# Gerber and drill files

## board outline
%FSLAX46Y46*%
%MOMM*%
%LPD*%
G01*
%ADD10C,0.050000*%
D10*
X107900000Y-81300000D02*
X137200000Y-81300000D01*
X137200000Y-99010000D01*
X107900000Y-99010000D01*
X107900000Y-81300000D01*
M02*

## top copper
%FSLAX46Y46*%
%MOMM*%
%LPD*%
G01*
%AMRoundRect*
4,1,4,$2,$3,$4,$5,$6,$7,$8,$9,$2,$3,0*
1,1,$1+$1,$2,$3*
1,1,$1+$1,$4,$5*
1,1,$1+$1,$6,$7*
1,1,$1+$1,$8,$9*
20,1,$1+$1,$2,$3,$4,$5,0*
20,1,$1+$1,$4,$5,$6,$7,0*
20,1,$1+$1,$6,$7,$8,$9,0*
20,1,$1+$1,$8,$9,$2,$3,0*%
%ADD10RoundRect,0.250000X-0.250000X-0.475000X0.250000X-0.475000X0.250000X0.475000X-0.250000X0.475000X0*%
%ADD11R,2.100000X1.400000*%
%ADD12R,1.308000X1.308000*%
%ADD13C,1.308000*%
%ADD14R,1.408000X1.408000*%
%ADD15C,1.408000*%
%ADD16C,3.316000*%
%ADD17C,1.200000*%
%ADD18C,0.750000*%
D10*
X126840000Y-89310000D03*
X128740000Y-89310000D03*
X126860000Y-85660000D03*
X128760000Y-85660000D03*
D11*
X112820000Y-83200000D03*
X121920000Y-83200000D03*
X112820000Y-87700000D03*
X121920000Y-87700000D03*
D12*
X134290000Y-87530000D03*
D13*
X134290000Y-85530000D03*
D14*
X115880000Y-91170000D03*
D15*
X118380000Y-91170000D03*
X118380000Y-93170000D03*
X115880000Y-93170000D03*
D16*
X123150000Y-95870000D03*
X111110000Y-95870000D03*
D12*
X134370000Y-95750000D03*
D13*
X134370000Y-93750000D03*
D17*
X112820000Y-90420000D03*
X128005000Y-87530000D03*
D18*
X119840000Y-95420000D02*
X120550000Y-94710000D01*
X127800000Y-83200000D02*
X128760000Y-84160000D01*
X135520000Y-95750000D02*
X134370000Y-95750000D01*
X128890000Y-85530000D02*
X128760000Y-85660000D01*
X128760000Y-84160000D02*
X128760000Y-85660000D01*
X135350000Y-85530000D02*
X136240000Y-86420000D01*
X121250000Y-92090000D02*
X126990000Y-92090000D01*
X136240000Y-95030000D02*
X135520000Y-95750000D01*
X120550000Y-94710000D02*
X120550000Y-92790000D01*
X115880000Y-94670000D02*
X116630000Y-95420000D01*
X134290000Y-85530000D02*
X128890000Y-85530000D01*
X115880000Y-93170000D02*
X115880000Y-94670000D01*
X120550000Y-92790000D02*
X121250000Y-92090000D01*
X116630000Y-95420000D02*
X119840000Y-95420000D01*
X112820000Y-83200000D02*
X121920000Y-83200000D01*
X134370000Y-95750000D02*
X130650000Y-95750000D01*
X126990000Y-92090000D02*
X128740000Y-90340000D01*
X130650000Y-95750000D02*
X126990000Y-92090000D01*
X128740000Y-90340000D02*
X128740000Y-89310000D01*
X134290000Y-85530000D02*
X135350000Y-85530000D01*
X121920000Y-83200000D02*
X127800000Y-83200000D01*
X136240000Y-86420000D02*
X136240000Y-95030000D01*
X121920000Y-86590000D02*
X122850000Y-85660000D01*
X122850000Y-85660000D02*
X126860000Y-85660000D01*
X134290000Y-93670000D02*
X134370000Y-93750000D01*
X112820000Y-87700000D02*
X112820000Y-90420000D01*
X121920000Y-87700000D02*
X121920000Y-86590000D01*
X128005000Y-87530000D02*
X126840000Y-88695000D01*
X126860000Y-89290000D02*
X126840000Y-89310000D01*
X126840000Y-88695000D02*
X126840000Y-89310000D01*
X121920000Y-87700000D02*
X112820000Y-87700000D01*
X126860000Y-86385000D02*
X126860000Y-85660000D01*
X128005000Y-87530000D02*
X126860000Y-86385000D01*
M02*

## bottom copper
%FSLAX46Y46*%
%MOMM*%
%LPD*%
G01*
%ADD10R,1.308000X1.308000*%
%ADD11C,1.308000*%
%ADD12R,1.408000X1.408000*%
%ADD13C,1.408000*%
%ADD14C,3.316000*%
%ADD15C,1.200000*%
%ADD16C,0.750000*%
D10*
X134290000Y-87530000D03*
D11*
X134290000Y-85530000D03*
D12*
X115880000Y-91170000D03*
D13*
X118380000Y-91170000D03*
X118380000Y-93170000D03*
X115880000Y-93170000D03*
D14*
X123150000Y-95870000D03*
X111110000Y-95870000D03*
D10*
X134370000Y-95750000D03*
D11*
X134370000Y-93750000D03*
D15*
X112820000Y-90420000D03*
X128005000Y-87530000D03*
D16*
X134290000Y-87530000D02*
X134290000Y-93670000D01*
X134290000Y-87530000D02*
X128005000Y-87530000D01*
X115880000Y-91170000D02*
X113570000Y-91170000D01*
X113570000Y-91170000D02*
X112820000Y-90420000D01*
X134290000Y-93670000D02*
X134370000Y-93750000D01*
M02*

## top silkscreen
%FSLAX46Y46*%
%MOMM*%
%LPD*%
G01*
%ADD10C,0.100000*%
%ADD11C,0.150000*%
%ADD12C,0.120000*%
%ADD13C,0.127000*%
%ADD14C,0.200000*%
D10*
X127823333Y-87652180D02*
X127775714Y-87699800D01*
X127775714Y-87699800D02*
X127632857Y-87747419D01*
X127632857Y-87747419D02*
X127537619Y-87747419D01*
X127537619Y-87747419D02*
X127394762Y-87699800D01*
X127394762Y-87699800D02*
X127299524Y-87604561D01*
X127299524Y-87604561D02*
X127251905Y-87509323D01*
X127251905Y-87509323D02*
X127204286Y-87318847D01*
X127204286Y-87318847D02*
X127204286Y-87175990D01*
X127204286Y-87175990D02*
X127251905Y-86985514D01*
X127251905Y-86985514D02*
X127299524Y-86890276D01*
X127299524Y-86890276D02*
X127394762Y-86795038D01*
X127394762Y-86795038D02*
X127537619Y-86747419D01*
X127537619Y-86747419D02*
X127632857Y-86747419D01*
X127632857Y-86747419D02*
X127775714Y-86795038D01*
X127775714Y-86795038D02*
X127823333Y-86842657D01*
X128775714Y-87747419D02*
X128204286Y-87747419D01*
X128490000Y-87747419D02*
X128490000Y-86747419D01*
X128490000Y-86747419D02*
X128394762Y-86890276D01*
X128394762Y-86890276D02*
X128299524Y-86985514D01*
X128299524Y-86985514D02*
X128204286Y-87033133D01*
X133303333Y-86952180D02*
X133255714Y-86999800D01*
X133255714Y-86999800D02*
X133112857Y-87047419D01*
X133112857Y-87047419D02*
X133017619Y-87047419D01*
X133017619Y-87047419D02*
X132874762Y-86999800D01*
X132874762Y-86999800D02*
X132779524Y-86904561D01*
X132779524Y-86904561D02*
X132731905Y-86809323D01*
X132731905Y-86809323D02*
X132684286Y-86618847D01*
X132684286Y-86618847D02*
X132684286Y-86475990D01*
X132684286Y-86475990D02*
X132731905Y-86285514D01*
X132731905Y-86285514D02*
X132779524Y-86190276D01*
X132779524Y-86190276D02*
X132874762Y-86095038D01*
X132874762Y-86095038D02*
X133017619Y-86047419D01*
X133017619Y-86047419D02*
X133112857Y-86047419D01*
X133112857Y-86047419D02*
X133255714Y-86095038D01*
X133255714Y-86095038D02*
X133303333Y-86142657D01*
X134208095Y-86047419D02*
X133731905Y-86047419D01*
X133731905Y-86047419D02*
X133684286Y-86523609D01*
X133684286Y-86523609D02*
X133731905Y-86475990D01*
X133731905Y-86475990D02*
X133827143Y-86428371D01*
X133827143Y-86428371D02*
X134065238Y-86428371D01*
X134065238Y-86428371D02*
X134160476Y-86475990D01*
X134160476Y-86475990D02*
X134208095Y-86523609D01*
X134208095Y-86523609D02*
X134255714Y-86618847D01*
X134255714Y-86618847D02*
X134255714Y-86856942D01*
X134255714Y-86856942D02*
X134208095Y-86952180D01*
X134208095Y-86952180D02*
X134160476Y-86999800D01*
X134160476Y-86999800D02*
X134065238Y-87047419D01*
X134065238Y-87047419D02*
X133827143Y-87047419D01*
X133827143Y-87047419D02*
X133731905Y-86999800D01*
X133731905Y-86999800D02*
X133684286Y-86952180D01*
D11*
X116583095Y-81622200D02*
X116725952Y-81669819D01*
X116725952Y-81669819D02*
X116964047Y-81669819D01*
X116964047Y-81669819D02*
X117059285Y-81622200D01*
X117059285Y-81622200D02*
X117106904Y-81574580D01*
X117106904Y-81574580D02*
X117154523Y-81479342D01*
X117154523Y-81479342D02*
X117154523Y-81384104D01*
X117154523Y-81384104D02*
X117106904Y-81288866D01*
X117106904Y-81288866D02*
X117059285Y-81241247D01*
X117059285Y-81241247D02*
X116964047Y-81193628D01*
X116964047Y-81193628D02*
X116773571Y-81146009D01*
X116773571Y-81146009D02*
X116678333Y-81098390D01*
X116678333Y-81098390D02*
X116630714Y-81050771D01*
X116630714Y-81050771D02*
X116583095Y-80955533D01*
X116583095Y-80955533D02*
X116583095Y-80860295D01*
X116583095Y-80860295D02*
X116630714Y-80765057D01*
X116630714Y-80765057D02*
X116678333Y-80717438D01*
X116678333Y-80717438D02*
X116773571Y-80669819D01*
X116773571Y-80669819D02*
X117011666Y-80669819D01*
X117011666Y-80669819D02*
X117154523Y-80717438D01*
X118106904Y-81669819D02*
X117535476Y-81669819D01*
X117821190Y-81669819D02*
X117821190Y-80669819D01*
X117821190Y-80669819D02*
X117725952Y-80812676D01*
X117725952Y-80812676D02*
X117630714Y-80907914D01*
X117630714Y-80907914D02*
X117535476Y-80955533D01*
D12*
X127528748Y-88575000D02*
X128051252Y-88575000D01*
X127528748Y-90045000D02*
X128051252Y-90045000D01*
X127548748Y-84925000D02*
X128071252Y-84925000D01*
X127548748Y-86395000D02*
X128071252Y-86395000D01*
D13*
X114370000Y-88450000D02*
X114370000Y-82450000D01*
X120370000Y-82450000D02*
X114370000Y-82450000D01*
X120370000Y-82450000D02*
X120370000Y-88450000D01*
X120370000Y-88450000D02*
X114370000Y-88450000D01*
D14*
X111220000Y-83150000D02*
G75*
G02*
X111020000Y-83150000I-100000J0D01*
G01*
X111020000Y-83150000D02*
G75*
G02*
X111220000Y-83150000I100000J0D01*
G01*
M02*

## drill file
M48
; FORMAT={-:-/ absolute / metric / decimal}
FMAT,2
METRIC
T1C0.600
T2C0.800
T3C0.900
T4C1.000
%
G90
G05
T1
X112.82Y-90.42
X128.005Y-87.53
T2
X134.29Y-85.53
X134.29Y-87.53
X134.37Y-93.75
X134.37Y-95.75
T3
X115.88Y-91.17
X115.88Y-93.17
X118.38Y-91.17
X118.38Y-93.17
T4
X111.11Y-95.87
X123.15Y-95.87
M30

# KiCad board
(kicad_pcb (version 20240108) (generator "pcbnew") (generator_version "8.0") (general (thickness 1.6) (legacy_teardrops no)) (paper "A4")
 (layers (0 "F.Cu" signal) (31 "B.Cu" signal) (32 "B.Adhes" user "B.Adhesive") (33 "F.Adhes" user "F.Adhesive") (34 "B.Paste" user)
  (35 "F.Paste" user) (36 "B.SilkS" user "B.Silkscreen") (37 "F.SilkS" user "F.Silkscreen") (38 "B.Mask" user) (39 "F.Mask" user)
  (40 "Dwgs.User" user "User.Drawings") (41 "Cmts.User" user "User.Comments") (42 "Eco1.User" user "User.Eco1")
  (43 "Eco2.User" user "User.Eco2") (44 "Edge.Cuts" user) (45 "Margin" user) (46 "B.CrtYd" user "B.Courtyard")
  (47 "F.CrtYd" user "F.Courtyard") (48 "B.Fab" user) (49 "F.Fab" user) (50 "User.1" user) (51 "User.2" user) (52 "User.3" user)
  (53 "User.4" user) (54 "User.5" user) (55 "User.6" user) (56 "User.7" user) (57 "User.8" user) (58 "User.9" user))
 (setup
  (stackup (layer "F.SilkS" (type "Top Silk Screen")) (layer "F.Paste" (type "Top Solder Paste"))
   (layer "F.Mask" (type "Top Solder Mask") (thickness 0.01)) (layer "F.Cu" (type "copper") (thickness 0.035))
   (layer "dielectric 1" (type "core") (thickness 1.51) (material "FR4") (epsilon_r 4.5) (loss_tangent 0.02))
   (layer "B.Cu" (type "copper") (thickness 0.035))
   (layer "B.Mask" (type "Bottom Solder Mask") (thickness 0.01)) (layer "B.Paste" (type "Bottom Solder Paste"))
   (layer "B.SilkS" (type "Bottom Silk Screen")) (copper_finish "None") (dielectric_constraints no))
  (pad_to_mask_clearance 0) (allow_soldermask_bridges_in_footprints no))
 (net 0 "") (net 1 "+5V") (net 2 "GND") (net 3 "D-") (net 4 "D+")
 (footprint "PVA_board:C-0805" (layer "F.Cu") (at 127.79 89.31)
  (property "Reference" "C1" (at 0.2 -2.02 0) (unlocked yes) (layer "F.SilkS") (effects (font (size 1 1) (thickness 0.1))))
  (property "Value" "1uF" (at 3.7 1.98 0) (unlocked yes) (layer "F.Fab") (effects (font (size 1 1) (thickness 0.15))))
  (fp_line (start -0.261252 -0.735) (end 0.261252 -0.735) (stroke (width 0.12) (type solid)) (layer "F.SilkS"))
  (fp_line (start -0.261252 0.735) (end 0.261252 0.735) (stroke (width 0.12) (type solid)) (layer "F.SilkS"))
  (pad "1" smd roundrect (at -0.95 0) (size 1 1.45) (layers "F.Cu" "F.Paste" "F.Mask") (roundrect_rratio 0.25) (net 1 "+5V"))
  (pad "2" smd roundrect (at 0.95 0) (size 1 1.45) (layers "F.Cu" "F.Paste" "F.Mask") (roundrect_rratio 0.25) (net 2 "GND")))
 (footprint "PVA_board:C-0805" (layer "F.Cu") (at 127.81 85.66)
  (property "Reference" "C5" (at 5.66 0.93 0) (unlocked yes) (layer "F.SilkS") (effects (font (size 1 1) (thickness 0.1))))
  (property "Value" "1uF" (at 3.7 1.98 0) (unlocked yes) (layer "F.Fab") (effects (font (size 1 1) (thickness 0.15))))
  (fp_line (start -0.261252 -0.735) (end 0.261252 -0.735) (stroke (width 0.12) (type solid)) (layer "F.SilkS"))
  (fp_line (start -0.261252 0.735) (end 0.261252 0.735) (stroke (width 0.12) (type solid)) (layer "F.SilkS"))
  (pad "1" smd roundrect (at -0.95 0) (size 1 1.45) (layers "F.Cu" "F.Paste" "F.Mask") (roundrect_rratio 0.25) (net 1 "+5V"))
  (pad "2" smd roundrect (at 0.95 0) (size 1 1.45) (layers "F.Cu" "F.Paste" "F.Mask") (roundrect_rratio 0.25) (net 2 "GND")))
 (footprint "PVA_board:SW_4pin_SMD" (layer "F.Cu") (at 117.37 85.45)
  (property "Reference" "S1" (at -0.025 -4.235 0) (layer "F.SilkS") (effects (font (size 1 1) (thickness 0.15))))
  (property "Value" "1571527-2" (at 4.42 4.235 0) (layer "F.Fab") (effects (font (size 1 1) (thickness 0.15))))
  (fp_line (start -3 3) (end -3 -3) (stroke (width 0.127) (type solid)) (layer "F.SilkS"))
  (fp_line (start 3 -3) (end -3 -3) (stroke (width 0.127) (type solid)) (layer "F.SilkS"))
  (fp_line (start 3 -3) (end 3 3) (stroke (width 0.127) (type solid)) (layer "F.SilkS"))
  (fp_line (start 3 3) (end -3 3) (stroke (width 0.127) (type solid)) (layer "F.SilkS"))
  (fp_circle (center -6.25 -2.3) (end -6.15 -2.3) (stroke (width 0.2) (type solid)) (fill none) (layer "F.SilkS"))
  (pad "1" smd rect (at -4.55 -2.25) (size 2.1 1.4) (layers "F.Cu" "F.Paste" "F.Mask") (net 2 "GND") (solder_mask_margin 0.102))
  (pad "2" smd rect (at 4.55 -2.25) (size 2.1 1.4) (layers "F.Cu" "F.Paste" "F.Mask") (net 2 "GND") (solder_mask_margin 0.102))
  (pad "3" smd rect (at -4.55 2.25) (size 2.1 1.4) (layers "F.Cu" "F.Paste" "F.Mask") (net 1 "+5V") (solder_mask_margin 0.102))
  (pad "4" smd rect (at 4.55 2.25) (size 2.1 1.4) (layers "F.Cu" "F.Paste" "F.Mask") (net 1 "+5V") (solder_mask_margin 0.102)))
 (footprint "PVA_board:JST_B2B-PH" (layer "B.Cu") (at 134.29 86.53 -90)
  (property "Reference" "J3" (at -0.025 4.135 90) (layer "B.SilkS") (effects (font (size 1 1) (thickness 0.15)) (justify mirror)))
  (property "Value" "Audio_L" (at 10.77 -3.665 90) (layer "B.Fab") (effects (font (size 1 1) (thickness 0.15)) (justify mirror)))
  (pad "1" thru_hole rect (at 1 0 270) (size 1.308 1.308) (drill 0.8) (layers "*.Cu" "*.Mask") (remove_unused_layers no) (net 1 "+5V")
   (solder_mask_margin 0.102))
  (pad "2" thru_hole circle (at -1 0 270) (size 1.308 1.308) (drill 0.8) (layers "*.Cu" "*.Mask") (remove_unused_layers no) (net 2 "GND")
   (solder_mask_margin 0.102)))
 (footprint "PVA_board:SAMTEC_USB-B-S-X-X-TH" (layer "B.Cu") (at 117.13 98.87 180)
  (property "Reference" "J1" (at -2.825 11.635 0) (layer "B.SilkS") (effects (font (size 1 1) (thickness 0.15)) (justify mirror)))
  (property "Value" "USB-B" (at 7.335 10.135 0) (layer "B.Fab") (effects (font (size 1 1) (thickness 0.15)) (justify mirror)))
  (pad "1" thru_hole rect (at 1.25 7.7 180) (size 1.408 1.408) (drill 0.9) (layers "*.Cu" "*.Mask") (remove_unused_layers no) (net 1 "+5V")
   (solder_mask_margin 0.102))
  (pad "2" thru_hole circle (at -1.25 7.7 180) (size 1.408 1.408) (drill 0.9) (layers "*.Cu" "*.Mask") (remove_unused_layers no)
   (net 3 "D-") (solder_mask_margin 0.102))
  (pad "3" thru_hole circle (at -1.25 5.7 180) (size 1.408 1.408) (drill 0.9) (layers "*.Cu" "*.Mask") (remove_unused_layers no)
   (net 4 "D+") (solder_mask_margin 0.102))
  (pad "4" thru_hole circle (at 1.25 5.7 180) (size 1.408 1.408) (drill 0.9) (layers "*.Cu" "*.Mask") (remove_unused_layers no)
   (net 2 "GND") (solder_mask_margin 0.102))
  (pad "S1" thru_hole circle (at -6.02 3 180) (size 3.316 3.316) (drill 1) (layers "*.Cu" "*.Mask") (remove_unused_layers no) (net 2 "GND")
   (solder_mask_margin 0.102))
  (pad "S2" thru_hole circle (at 6.02 3 180) (size 3.316 3.316) (drill 1) (layers "*.Cu" "*.Mask") (remove_unused_layers no) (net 2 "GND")
   (solder_mask_margin 0.102)))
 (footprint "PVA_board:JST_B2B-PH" (layer "B.Cu") (at 134.37 94.75 -90)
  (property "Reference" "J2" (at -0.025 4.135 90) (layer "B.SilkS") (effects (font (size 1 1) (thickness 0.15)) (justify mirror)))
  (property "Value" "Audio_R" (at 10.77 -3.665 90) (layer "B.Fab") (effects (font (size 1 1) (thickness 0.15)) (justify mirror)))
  (pad "1" thru_hole rect (at 1 0 270) (size 1.308 1.308) (drill 0.8) (layers "*.Cu" "*.Mask") (remove_unused_layers no) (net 2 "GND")
   (solder_mask_margin 0.102))
  (pad "2" thru_hole circle (at -1 0 270) (size 1.308 1.308) (drill 0.8) (layers "*.Cu" "*.Mask") (remove_unused_layers no) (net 1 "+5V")
   (solder_mask_margin 0.102)))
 (gr_rect (start 107.9 81.3) (end 137.2 99.01) (stroke (width 0.05) (type default)) (fill none) (layer "Edge.Cuts"))
 (segment (start 119.84 95.42) (end 120.55 94.71) (width 0.75) (layer "F.Cu") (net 2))
 (segment (start 127.8 83.2) (end 128.76 84.16) (width 0.75) (layer "F.Cu") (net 2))
 (segment (start 135.52 95.75) (end 134.37 95.75) (width 0.75) (layer "F.Cu") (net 2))
 (segment (start 128.89 85.53) (end 128.76 85.66) (width 0.75) (layer "F.Cu") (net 2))
 (segment (start 128.76 84.16) (end 128.76 85.66) (width 0.75) (layer "F.Cu") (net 2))
 (segment (start 135.35 85.53) (end 136.24 86.42) (width 0.75) (layer "F.Cu") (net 2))
 (segment (start 121.25 92.09) (end 126.99 92.09) (width 0.75) (layer "F.Cu") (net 2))
 (segment (start 136.24 95.03) (end 135.52 95.75) (width 0.75) (layer "F.Cu") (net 2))
 (segment (start 120.55 94.71) (end 120.55 92.79) (width 0.75) (layer "F.Cu") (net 2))
 (segment (start 115.88 94.67) (end 116.63 95.42) (width 0.75) (layer "F.Cu") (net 2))
 (segment (start 134.29 85.53) (end 128.89 85.53) (width 0.75) (layer "F.Cu") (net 2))
 (segment (start 115.88 93.17) (end 115.88 94.67) (width 0.75) (layer "F.Cu") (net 2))
 (segment (start 120.55 92.79) (end 121.25 92.09) (width 0.75) (layer "F.Cu") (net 2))
 (segment (start 116.63 95.42) (end 119.84 95.42) (width 0.75) (layer "F.Cu") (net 2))
 (segment (start 112.82 83.2) (end 121.92 83.2) (width 0.75) (layer "F.Cu") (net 2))
 (segment (start 134.37 95.75) (end 130.65 95.75) (width 0.75) (layer "F.Cu") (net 2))
 (segment (start 126.99 92.09) (end 128.74 90.34) (width 0.75) (layer "F.Cu") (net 2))
 (segment (start 130.65 95.75) (end 126.99 92.09) (width 0.75) (layer "F.Cu") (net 2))
 (segment (start 128.74 90.34) (end 128.74 89.31) (width 0.75) (layer "F.Cu") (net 2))
 (segment (start 134.29 85.53) (end 135.35 85.53) (width 0.75) (layer "F.Cu") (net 2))
 (segment (start 121.92 83.2) (end 127.8 83.2) (width 0.75) (layer "F.Cu") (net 2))
 (segment (start 136.24 86.42) (end 136.24 95.03) (width 0.75) (layer "F.Cu") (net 2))
 (segment (start 121.92 86.59) (end 122.85 85.66) (width 0.75) (layer "F.Cu") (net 1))
 (segment (start 122.85 85.66) (end 126.86 85.66) (width 0.75) (layer "F.Cu") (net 1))
 (segment (start 134.29 93.67) (end 134.37 93.75) (width 0.75) (layer "F.Cu") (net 1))
 (segment (start 112.82 87.7) (end 112.82 90.42) (width 0.75) (layer "F.Cu") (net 1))
 (segment (start 121.92 87.7) (end 121.92 86.59) (width 0.75) (layer "F.Cu") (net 1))
 (segment (start 128.005 87.53) (end 126.84 88.695) (width 0.75) (layer "F.Cu") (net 1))
 (segment (start 126.86 89.29) (end 126.84 89.31) (width 0.75) (layer "F.Cu") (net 1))
 (segment (start 126.84 88.695) (end 126.84 89.31) (width 0.75) (layer "F.Cu") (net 1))
 (segment (start 121.92 87.7) (end 112.82 87.7) (width 0.75) (layer "F.Cu") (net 1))
 (segment (start 126.86 86.385) (end 126.86 85.66) (width 0.75) (layer "F.Cu") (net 1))
 (segment (start 128.005 87.53) (end 126.86 86.385) (width 0.75) (layer "F.Cu") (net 1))
 (via (at 112.82 90.42) (size 1.2) (drill 0.6) (layers "F.Cu" "B.Cu") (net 1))
 (via (at 128.005 87.53) (size 1.2) (drill 0.6) (layers "F.Cu" "B.Cu") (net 1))
 (segment (start 134.29 87.53) (end 134.29 93.67) (width 0.75) (layer "B.Cu") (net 1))
 (segment (start 134.29 87.53) (end 128.005 87.53) (width 0.75) (layer "B.Cu") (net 1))
 (segment (start 115.88 91.17) (end 113.57 91.17) (width 0.75) (layer "B.Cu") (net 1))
 (segment (start 113.57 91.17) (end 112.82 90.42) (width 0.75) (layer "B.Cu") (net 1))
 (segment (start 134.29 93.67) (end 134.37 93.75) (width 0.75) (layer "B.Cu") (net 1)))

